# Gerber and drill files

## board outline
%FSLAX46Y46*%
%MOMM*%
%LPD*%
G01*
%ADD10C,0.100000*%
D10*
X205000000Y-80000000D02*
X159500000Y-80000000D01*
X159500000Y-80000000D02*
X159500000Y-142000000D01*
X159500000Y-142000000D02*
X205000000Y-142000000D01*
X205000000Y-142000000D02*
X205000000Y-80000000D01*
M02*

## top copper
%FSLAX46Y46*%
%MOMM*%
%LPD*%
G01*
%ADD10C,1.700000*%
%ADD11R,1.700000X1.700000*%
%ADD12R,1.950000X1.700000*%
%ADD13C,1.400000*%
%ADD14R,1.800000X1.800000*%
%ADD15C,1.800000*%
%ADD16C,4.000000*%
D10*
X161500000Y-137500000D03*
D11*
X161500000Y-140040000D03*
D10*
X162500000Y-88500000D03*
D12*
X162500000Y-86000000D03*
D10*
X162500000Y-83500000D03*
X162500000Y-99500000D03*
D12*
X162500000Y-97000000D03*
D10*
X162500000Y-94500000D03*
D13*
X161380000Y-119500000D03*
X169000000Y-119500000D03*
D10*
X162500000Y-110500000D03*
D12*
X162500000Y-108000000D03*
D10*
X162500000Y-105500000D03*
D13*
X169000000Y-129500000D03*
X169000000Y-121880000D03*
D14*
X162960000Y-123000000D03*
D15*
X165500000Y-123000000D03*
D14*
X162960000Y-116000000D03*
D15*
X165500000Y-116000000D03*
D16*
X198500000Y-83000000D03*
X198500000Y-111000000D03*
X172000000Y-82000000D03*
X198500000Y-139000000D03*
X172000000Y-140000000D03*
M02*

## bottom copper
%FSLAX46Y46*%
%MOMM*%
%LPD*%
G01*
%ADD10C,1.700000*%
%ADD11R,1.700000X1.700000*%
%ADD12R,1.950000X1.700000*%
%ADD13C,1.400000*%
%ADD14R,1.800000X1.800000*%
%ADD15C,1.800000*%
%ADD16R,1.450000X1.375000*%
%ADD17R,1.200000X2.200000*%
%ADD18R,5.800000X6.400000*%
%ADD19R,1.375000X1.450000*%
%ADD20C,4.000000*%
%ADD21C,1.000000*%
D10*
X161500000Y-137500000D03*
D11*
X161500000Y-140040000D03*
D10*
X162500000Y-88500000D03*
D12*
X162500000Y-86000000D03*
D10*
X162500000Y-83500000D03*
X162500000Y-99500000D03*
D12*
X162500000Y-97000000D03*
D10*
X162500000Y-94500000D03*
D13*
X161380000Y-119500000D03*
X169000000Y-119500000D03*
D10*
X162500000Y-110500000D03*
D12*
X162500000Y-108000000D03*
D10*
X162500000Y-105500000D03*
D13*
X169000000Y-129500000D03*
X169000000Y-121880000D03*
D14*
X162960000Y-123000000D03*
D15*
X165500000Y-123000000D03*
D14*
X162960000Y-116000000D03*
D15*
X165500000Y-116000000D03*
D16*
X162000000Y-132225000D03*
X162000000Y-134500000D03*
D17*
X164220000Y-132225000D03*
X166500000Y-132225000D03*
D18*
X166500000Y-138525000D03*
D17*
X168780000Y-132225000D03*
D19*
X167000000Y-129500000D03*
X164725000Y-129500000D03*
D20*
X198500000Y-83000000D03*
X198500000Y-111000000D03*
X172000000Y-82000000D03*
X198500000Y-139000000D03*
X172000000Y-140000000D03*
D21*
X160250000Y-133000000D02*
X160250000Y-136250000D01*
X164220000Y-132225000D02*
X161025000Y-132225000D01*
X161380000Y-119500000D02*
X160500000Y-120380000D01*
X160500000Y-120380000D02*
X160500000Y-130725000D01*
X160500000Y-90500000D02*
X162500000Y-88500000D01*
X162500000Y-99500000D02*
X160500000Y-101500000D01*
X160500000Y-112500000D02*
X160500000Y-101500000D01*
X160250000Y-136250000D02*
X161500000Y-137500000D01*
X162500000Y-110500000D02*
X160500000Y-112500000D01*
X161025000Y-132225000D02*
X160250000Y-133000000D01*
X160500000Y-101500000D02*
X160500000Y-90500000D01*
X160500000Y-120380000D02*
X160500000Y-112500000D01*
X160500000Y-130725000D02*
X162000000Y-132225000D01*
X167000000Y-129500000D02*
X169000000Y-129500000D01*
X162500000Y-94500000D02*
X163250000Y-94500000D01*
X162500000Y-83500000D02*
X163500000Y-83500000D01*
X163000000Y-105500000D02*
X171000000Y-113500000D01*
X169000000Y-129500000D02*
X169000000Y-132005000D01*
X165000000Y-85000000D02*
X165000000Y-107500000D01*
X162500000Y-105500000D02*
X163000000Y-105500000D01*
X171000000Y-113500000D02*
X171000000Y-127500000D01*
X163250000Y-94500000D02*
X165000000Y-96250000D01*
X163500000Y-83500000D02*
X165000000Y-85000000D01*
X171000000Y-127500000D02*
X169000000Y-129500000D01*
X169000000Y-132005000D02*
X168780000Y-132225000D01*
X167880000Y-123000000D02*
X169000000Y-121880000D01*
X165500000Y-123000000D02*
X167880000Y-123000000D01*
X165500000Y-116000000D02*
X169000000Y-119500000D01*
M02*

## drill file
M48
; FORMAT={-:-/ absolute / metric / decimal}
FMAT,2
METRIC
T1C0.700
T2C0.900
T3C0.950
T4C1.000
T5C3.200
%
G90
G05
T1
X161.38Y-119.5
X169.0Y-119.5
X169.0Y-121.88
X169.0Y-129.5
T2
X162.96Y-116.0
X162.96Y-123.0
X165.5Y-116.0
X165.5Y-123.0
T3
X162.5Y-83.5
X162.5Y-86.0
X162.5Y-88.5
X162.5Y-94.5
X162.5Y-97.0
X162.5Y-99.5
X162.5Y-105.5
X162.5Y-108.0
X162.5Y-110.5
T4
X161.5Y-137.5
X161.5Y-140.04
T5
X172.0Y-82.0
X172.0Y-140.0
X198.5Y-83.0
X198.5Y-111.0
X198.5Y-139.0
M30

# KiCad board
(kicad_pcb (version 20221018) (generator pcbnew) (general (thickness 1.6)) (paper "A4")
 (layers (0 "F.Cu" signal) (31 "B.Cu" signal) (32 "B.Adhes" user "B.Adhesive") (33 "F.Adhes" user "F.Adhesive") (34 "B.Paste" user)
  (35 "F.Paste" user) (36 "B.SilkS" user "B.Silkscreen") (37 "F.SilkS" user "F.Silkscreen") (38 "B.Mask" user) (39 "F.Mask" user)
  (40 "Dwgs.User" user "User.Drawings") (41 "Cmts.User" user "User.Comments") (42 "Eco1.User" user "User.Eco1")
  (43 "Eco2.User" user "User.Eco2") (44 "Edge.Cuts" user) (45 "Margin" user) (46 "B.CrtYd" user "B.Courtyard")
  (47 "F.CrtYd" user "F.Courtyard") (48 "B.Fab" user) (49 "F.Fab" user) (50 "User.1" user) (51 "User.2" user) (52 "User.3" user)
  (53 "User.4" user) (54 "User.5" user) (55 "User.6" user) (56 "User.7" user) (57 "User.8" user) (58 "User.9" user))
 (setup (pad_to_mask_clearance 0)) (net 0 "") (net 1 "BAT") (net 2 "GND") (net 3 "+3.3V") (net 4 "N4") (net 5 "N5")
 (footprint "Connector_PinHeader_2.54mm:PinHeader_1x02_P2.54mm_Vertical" (layer "F.Cu") (at 161.5 137.5)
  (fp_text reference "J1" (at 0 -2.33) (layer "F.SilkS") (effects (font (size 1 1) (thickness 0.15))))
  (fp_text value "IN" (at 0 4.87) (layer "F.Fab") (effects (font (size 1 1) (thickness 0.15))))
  (pad "1" thru_hole circle (at 0 0) (size 1.7 1.7) (drill 1) (layers "*.Cu" "*.Mask") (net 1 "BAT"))
  (pad "2" thru_hole rect (at 0 2.54) (size 1.7 1.7) (drill 1) (layers "*.Cu" "*.Mask") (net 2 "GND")))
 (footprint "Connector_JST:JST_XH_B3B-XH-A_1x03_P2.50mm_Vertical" (layer "F.Cu") (at 162.5 88.5 90)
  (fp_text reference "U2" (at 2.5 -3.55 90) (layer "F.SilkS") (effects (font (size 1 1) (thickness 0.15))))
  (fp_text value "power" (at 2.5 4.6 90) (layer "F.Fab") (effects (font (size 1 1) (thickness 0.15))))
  (pad "1" thru_hole circle (at 0 0 90) (size 1.7 1.7) (drill 0.95) (layers "*.Cu" "*.Mask" "Dwgs.User") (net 1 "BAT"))
  (pad "2" thru_hole rect (at 2.5 0 90) (size 1.7 1.95) (drill 0.95) (layers "*.Cu" "*.Mask") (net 2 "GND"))
  (pad "3" thru_hole circle (at 5 0 90) (size 1.7 1.7) (drill 0.95) (layers "*.Cu" "*.Mask") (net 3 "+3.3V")))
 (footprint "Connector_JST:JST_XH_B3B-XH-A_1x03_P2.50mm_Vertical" (layer "F.Cu") (at 162.5 99.5 90)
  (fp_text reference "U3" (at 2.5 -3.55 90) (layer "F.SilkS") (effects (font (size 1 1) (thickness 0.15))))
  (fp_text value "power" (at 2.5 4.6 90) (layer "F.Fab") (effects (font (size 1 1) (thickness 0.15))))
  (pad "1" thru_hole circle (at 0 0 90) (size 1.7 1.7) (drill 0.95) (layers "*.Cu" "*.Mask") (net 1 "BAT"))
  (pad "2" thru_hole rect (at 2.5 0 90) (size 1.7 1.95) (drill 0.95) (layers "*.Cu" "*.Mask") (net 2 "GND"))
  (pad "3" thru_hole circle (at 5 0 90) (size 1.7 1.7) (drill 0.95) (layers "*.Cu" "*.Mask") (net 3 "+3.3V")))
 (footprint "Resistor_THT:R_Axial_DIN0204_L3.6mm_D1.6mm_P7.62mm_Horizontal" (layer "F.Cu") (at 161.38 119.5)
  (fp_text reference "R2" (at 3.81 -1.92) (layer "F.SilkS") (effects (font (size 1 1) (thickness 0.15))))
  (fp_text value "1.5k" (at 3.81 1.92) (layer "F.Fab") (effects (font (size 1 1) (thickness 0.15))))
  (pad "1" thru_hole circle (at 0 0) (size 1.4 1.4) (drill 0.7) (layers "*.Cu" "*.Mask") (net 1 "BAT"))
  (pad "2" thru_hole circle (at 7.62 0) (size 1.4 1.4) (drill 0.7) (layers "*.Cu" "*.Mask") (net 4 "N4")))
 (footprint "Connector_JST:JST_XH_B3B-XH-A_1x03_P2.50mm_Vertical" (layer "F.Cu") (at 162.5 110.5 90)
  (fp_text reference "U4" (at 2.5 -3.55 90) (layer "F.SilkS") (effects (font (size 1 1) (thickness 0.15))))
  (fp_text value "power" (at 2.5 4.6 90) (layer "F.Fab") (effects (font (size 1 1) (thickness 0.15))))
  (pad "1" thru_hole circle (at 0 0 90) (size 1.7 1.7) (drill 0.95) (layers "*.Cu" "*.Mask") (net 1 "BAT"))
  (pad "2" thru_hole rect (at 2.5 0 90) (size 1.7 1.95) (drill 0.95) (layers "*.Cu" "*.Mask") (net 2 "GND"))
  (pad "3" thru_hole circle (at 5 0 90) (size 1.7 1.7) (drill 0.95) (layers "*.Cu" "*.Mask") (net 3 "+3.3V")))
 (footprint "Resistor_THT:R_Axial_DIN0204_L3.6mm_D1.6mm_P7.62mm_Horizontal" (layer "F.Cu") (at 169 129.5 90)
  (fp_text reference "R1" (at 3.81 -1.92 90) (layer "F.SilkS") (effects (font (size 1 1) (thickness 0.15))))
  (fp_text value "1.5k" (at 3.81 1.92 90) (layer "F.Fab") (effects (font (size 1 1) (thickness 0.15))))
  (pad "1" thru_hole circle (at 0 0 90) (size 1.4 1.4) (drill 0.7) (layers "*.Cu" "*.Mask") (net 3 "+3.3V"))
  (pad "2" thru_hole circle (at 7.62 0 90) (size 1.4 1.4) (drill 0.7) (layers "*.Cu" "*.Mask") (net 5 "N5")))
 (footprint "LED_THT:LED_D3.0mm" (layer "F.Cu") (at 162.96 123)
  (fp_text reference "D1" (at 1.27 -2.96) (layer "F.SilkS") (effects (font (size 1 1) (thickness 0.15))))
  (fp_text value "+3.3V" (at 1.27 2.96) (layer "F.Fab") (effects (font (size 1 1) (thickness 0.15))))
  (pad "1" thru_hole rect (at 0 0) (size 1.8 1.8) (drill 0.9) (layers "*.Cu" "*.Mask") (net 2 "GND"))
  (pad "2" thru_hole circle (at 2.54 0) (size 1.8 1.8) (drill 0.9) (layers "*.Cu" "*.Mask") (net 5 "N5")))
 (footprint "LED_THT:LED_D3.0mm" (layer "F.Cu") (at 162.96 116)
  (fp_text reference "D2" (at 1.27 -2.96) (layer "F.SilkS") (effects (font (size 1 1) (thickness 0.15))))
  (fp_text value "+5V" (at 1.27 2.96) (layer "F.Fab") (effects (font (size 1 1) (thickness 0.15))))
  (pad "1" thru_hole rect (at 0 0) (size 1.8 1.8) (drill 0.9) (layers "*.Cu" "*.Mask") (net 2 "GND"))
  (pad "2" thru_hole circle (at 2.54 0) (size 1.8 1.8) (drill 0.9) (layers "*.Cu" "*.Mask") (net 4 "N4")))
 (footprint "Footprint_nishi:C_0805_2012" (layer "B.Cu") (at 162 133.3625 -90)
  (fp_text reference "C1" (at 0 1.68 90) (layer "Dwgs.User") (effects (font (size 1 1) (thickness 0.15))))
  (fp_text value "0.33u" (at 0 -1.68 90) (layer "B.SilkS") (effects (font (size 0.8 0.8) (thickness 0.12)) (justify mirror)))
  (pad "1" smd rect (at -1.1375 0 270) (size 1.375 1.45) (layers "B.Cu" "B.Paste" "B.Mask") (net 1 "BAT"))
  (pad "2" smd rect (at 1.1375 0 270) (size 1.375 1.45) (layers "B.Cu" "B.Paste" "B.Mask") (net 2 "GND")))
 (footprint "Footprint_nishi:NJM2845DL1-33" (layer "B.Cu") (at 166.5 136.425 -90)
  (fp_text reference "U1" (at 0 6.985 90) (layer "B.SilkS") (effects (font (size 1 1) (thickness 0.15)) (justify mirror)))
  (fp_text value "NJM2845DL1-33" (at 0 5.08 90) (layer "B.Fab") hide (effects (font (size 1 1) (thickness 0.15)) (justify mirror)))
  (pad "1" smd rect (at -4.2 2.28 270) (size 2.2 1.2) (layers "B.Cu" "B.Paste" "B.Mask") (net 1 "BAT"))
  (pad "2" smd rect (at -4.2 0 270) (size 2.2 1.2) (layers "B.Cu" "B.Paste" "B.Mask") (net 2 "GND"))
  (pad "2" smd rect (at 2.1 0 270) (size 6.4 5.8) (layers "B.Cu" "B.Paste" "B.Mask") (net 2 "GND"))
  (pad "3" smd rect (at -4.2 -2.28 270) (size 2.2 1.2) (layers "B.Cu" "B.Paste" "B.Mask") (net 3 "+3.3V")))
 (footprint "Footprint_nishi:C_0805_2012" (layer "B.Cu") (at 165.8625 129.5 180)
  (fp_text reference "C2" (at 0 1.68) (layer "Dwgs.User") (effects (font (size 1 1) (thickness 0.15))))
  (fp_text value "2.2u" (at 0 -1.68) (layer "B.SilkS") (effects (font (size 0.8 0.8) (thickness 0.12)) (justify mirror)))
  (pad "1" smd rect (at -1.1375 0 180) (size 1.375 1.45) (layers "B.Cu" "B.Paste" "B.Mask") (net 3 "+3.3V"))
  (pad "2" smd rect (at 1.1375 0 180) (size 1.375 1.45) (layers "B.Cu" "B.Paste" "B.Mask") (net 2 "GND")))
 (gr_line (start 205 80) (end 159.5 80) (stroke (width 0.1) (type default)) (layer "Edge.Cuts"))
 (gr_line (start 159.5 80) (end 159.5 142) (stroke (width 0.1) (type default)) (layer "Edge.Cuts"))
 (gr_line (start 159.5 142) (end 205 142) (stroke (width 0.1) (type default)) (layer "Edge.Cuts"))
 (gr_line (start 205 142) (end 205 80) (stroke (width 0.1) (type default)) (layer "Edge.Cuts"))
 (via (at 198.5 83) (size 4) (drill 3.2) (layers "F.Cu" "B.Cu") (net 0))
 (via (at 198.5 111) (size 4) (drill 3.2) (layers "F.Cu" "B.Cu") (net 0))
 (via (at 172 82) (size 4) (drill 3.2) (layers "F.Cu" "B.Cu") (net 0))
 (via (at 198.5 139) (size 4) (drill 3.2) (layers "F.Cu" "B.Cu") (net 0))
 (via (at 172 140) (size 4) (drill 3.2) (layers "F.Cu" "B.Cu") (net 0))
 (segment (start 160.25 133) (end 160.25 136.25) (width 1) (layer "B.Cu") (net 1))
 (segment (start 164.22 132.225) (end 161.025 132.225) (width 1) (layer "B.Cu") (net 1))
 (segment (start 161.38 119.5) (end 160.5 120.38) (width 1) (layer "B.Cu") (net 1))
 (segment (start 160.5 120.38) (end 160.5 130.725) (width 1) (layer "B.Cu") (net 1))
 (segment (start 160.5 90.5) (end 162.5 88.5) (width 1) (layer "B.Cu") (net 1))
 (segment (start 162.5 99.5) (end 160.5 101.5) (width 1) (layer "B.Cu") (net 1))
 (segment (start 160.5 112.5) (end 160.5 101.5) (width 1) (layer "B.Cu") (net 1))
 (segment (start 160.25 136.25) (end 161.5 137.5) (width 1) (layer "B.Cu") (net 1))
 (segment (start 162.5 110.5) (end 160.5 112.5) (width 1) (layer "B.Cu") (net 1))
 (segment (start 161.025 132.225) (end 160.25 133) (width 1) (layer "B.Cu") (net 1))
 (segment (start 160.5 101.5) (end 160.5 90.5) (width 1) (layer "B.Cu") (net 1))
 (segment (start 160.5 120.38) (end 160.5 112.5) (width 1) (layer "B.Cu") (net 1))
 (segment (start 160.5 130.725) (end 162 132.225) (width 1) (layer "B.Cu") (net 1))
 (segment (start 167 129.5) (end 169 129.5) (width 1) (layer "B.Cu") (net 3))
 (segment (start 162.5 94.5) (end 163.25 94.5) (width 1) (layer "B.Cu") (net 3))
 (segment (start 162.5 83.5) (end 163.5 83.5) (width 1) (layer "B.Cu") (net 3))
 (segment (start 163 105.5) (end 171 113.5) (width 1) (layer "B.Cu") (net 3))
 (segment (start 169 129.5) (end 169 132.005) (width 1) (layer "B.Cu") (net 3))
 (segment (start 165 85) (end 165 107.5) (width 1) (layer "B.Cu") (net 3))
 (segment (start 162.5 105.5) (end 163 105.5) (width 1) (layer "B.Cu") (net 3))
 (segment (start 171 113.5) (end 171 127.5) (width 1) (layer "B.Cu") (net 3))
 (segment (start 163.25 94.5) (end 165 96.25) (width 1) (layer "B.Cu") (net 3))
 (segment (start 163.5 83.5) (end 165 85) (width 1) (layer "B.Cu") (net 3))
 (segment (start 171 127.5) (end 169 129.5) (width 1) (layer "B.Cu") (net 3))
 (segment (start 169 132.005) (end 168.78 132.225) (width 1) (layer "B.Cu") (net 3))
 (segment (start 167.88 123) (end 169 121.88) (width 1) (layer "B.Cu") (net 5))
 (segment (start 165.5 123) (end 167.88 123) (width 1) (layer "B.Cu") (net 5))
 (segment (start 165.5 116) (end 169 119.5) (width 1) (layer "B.Cu") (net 4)))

